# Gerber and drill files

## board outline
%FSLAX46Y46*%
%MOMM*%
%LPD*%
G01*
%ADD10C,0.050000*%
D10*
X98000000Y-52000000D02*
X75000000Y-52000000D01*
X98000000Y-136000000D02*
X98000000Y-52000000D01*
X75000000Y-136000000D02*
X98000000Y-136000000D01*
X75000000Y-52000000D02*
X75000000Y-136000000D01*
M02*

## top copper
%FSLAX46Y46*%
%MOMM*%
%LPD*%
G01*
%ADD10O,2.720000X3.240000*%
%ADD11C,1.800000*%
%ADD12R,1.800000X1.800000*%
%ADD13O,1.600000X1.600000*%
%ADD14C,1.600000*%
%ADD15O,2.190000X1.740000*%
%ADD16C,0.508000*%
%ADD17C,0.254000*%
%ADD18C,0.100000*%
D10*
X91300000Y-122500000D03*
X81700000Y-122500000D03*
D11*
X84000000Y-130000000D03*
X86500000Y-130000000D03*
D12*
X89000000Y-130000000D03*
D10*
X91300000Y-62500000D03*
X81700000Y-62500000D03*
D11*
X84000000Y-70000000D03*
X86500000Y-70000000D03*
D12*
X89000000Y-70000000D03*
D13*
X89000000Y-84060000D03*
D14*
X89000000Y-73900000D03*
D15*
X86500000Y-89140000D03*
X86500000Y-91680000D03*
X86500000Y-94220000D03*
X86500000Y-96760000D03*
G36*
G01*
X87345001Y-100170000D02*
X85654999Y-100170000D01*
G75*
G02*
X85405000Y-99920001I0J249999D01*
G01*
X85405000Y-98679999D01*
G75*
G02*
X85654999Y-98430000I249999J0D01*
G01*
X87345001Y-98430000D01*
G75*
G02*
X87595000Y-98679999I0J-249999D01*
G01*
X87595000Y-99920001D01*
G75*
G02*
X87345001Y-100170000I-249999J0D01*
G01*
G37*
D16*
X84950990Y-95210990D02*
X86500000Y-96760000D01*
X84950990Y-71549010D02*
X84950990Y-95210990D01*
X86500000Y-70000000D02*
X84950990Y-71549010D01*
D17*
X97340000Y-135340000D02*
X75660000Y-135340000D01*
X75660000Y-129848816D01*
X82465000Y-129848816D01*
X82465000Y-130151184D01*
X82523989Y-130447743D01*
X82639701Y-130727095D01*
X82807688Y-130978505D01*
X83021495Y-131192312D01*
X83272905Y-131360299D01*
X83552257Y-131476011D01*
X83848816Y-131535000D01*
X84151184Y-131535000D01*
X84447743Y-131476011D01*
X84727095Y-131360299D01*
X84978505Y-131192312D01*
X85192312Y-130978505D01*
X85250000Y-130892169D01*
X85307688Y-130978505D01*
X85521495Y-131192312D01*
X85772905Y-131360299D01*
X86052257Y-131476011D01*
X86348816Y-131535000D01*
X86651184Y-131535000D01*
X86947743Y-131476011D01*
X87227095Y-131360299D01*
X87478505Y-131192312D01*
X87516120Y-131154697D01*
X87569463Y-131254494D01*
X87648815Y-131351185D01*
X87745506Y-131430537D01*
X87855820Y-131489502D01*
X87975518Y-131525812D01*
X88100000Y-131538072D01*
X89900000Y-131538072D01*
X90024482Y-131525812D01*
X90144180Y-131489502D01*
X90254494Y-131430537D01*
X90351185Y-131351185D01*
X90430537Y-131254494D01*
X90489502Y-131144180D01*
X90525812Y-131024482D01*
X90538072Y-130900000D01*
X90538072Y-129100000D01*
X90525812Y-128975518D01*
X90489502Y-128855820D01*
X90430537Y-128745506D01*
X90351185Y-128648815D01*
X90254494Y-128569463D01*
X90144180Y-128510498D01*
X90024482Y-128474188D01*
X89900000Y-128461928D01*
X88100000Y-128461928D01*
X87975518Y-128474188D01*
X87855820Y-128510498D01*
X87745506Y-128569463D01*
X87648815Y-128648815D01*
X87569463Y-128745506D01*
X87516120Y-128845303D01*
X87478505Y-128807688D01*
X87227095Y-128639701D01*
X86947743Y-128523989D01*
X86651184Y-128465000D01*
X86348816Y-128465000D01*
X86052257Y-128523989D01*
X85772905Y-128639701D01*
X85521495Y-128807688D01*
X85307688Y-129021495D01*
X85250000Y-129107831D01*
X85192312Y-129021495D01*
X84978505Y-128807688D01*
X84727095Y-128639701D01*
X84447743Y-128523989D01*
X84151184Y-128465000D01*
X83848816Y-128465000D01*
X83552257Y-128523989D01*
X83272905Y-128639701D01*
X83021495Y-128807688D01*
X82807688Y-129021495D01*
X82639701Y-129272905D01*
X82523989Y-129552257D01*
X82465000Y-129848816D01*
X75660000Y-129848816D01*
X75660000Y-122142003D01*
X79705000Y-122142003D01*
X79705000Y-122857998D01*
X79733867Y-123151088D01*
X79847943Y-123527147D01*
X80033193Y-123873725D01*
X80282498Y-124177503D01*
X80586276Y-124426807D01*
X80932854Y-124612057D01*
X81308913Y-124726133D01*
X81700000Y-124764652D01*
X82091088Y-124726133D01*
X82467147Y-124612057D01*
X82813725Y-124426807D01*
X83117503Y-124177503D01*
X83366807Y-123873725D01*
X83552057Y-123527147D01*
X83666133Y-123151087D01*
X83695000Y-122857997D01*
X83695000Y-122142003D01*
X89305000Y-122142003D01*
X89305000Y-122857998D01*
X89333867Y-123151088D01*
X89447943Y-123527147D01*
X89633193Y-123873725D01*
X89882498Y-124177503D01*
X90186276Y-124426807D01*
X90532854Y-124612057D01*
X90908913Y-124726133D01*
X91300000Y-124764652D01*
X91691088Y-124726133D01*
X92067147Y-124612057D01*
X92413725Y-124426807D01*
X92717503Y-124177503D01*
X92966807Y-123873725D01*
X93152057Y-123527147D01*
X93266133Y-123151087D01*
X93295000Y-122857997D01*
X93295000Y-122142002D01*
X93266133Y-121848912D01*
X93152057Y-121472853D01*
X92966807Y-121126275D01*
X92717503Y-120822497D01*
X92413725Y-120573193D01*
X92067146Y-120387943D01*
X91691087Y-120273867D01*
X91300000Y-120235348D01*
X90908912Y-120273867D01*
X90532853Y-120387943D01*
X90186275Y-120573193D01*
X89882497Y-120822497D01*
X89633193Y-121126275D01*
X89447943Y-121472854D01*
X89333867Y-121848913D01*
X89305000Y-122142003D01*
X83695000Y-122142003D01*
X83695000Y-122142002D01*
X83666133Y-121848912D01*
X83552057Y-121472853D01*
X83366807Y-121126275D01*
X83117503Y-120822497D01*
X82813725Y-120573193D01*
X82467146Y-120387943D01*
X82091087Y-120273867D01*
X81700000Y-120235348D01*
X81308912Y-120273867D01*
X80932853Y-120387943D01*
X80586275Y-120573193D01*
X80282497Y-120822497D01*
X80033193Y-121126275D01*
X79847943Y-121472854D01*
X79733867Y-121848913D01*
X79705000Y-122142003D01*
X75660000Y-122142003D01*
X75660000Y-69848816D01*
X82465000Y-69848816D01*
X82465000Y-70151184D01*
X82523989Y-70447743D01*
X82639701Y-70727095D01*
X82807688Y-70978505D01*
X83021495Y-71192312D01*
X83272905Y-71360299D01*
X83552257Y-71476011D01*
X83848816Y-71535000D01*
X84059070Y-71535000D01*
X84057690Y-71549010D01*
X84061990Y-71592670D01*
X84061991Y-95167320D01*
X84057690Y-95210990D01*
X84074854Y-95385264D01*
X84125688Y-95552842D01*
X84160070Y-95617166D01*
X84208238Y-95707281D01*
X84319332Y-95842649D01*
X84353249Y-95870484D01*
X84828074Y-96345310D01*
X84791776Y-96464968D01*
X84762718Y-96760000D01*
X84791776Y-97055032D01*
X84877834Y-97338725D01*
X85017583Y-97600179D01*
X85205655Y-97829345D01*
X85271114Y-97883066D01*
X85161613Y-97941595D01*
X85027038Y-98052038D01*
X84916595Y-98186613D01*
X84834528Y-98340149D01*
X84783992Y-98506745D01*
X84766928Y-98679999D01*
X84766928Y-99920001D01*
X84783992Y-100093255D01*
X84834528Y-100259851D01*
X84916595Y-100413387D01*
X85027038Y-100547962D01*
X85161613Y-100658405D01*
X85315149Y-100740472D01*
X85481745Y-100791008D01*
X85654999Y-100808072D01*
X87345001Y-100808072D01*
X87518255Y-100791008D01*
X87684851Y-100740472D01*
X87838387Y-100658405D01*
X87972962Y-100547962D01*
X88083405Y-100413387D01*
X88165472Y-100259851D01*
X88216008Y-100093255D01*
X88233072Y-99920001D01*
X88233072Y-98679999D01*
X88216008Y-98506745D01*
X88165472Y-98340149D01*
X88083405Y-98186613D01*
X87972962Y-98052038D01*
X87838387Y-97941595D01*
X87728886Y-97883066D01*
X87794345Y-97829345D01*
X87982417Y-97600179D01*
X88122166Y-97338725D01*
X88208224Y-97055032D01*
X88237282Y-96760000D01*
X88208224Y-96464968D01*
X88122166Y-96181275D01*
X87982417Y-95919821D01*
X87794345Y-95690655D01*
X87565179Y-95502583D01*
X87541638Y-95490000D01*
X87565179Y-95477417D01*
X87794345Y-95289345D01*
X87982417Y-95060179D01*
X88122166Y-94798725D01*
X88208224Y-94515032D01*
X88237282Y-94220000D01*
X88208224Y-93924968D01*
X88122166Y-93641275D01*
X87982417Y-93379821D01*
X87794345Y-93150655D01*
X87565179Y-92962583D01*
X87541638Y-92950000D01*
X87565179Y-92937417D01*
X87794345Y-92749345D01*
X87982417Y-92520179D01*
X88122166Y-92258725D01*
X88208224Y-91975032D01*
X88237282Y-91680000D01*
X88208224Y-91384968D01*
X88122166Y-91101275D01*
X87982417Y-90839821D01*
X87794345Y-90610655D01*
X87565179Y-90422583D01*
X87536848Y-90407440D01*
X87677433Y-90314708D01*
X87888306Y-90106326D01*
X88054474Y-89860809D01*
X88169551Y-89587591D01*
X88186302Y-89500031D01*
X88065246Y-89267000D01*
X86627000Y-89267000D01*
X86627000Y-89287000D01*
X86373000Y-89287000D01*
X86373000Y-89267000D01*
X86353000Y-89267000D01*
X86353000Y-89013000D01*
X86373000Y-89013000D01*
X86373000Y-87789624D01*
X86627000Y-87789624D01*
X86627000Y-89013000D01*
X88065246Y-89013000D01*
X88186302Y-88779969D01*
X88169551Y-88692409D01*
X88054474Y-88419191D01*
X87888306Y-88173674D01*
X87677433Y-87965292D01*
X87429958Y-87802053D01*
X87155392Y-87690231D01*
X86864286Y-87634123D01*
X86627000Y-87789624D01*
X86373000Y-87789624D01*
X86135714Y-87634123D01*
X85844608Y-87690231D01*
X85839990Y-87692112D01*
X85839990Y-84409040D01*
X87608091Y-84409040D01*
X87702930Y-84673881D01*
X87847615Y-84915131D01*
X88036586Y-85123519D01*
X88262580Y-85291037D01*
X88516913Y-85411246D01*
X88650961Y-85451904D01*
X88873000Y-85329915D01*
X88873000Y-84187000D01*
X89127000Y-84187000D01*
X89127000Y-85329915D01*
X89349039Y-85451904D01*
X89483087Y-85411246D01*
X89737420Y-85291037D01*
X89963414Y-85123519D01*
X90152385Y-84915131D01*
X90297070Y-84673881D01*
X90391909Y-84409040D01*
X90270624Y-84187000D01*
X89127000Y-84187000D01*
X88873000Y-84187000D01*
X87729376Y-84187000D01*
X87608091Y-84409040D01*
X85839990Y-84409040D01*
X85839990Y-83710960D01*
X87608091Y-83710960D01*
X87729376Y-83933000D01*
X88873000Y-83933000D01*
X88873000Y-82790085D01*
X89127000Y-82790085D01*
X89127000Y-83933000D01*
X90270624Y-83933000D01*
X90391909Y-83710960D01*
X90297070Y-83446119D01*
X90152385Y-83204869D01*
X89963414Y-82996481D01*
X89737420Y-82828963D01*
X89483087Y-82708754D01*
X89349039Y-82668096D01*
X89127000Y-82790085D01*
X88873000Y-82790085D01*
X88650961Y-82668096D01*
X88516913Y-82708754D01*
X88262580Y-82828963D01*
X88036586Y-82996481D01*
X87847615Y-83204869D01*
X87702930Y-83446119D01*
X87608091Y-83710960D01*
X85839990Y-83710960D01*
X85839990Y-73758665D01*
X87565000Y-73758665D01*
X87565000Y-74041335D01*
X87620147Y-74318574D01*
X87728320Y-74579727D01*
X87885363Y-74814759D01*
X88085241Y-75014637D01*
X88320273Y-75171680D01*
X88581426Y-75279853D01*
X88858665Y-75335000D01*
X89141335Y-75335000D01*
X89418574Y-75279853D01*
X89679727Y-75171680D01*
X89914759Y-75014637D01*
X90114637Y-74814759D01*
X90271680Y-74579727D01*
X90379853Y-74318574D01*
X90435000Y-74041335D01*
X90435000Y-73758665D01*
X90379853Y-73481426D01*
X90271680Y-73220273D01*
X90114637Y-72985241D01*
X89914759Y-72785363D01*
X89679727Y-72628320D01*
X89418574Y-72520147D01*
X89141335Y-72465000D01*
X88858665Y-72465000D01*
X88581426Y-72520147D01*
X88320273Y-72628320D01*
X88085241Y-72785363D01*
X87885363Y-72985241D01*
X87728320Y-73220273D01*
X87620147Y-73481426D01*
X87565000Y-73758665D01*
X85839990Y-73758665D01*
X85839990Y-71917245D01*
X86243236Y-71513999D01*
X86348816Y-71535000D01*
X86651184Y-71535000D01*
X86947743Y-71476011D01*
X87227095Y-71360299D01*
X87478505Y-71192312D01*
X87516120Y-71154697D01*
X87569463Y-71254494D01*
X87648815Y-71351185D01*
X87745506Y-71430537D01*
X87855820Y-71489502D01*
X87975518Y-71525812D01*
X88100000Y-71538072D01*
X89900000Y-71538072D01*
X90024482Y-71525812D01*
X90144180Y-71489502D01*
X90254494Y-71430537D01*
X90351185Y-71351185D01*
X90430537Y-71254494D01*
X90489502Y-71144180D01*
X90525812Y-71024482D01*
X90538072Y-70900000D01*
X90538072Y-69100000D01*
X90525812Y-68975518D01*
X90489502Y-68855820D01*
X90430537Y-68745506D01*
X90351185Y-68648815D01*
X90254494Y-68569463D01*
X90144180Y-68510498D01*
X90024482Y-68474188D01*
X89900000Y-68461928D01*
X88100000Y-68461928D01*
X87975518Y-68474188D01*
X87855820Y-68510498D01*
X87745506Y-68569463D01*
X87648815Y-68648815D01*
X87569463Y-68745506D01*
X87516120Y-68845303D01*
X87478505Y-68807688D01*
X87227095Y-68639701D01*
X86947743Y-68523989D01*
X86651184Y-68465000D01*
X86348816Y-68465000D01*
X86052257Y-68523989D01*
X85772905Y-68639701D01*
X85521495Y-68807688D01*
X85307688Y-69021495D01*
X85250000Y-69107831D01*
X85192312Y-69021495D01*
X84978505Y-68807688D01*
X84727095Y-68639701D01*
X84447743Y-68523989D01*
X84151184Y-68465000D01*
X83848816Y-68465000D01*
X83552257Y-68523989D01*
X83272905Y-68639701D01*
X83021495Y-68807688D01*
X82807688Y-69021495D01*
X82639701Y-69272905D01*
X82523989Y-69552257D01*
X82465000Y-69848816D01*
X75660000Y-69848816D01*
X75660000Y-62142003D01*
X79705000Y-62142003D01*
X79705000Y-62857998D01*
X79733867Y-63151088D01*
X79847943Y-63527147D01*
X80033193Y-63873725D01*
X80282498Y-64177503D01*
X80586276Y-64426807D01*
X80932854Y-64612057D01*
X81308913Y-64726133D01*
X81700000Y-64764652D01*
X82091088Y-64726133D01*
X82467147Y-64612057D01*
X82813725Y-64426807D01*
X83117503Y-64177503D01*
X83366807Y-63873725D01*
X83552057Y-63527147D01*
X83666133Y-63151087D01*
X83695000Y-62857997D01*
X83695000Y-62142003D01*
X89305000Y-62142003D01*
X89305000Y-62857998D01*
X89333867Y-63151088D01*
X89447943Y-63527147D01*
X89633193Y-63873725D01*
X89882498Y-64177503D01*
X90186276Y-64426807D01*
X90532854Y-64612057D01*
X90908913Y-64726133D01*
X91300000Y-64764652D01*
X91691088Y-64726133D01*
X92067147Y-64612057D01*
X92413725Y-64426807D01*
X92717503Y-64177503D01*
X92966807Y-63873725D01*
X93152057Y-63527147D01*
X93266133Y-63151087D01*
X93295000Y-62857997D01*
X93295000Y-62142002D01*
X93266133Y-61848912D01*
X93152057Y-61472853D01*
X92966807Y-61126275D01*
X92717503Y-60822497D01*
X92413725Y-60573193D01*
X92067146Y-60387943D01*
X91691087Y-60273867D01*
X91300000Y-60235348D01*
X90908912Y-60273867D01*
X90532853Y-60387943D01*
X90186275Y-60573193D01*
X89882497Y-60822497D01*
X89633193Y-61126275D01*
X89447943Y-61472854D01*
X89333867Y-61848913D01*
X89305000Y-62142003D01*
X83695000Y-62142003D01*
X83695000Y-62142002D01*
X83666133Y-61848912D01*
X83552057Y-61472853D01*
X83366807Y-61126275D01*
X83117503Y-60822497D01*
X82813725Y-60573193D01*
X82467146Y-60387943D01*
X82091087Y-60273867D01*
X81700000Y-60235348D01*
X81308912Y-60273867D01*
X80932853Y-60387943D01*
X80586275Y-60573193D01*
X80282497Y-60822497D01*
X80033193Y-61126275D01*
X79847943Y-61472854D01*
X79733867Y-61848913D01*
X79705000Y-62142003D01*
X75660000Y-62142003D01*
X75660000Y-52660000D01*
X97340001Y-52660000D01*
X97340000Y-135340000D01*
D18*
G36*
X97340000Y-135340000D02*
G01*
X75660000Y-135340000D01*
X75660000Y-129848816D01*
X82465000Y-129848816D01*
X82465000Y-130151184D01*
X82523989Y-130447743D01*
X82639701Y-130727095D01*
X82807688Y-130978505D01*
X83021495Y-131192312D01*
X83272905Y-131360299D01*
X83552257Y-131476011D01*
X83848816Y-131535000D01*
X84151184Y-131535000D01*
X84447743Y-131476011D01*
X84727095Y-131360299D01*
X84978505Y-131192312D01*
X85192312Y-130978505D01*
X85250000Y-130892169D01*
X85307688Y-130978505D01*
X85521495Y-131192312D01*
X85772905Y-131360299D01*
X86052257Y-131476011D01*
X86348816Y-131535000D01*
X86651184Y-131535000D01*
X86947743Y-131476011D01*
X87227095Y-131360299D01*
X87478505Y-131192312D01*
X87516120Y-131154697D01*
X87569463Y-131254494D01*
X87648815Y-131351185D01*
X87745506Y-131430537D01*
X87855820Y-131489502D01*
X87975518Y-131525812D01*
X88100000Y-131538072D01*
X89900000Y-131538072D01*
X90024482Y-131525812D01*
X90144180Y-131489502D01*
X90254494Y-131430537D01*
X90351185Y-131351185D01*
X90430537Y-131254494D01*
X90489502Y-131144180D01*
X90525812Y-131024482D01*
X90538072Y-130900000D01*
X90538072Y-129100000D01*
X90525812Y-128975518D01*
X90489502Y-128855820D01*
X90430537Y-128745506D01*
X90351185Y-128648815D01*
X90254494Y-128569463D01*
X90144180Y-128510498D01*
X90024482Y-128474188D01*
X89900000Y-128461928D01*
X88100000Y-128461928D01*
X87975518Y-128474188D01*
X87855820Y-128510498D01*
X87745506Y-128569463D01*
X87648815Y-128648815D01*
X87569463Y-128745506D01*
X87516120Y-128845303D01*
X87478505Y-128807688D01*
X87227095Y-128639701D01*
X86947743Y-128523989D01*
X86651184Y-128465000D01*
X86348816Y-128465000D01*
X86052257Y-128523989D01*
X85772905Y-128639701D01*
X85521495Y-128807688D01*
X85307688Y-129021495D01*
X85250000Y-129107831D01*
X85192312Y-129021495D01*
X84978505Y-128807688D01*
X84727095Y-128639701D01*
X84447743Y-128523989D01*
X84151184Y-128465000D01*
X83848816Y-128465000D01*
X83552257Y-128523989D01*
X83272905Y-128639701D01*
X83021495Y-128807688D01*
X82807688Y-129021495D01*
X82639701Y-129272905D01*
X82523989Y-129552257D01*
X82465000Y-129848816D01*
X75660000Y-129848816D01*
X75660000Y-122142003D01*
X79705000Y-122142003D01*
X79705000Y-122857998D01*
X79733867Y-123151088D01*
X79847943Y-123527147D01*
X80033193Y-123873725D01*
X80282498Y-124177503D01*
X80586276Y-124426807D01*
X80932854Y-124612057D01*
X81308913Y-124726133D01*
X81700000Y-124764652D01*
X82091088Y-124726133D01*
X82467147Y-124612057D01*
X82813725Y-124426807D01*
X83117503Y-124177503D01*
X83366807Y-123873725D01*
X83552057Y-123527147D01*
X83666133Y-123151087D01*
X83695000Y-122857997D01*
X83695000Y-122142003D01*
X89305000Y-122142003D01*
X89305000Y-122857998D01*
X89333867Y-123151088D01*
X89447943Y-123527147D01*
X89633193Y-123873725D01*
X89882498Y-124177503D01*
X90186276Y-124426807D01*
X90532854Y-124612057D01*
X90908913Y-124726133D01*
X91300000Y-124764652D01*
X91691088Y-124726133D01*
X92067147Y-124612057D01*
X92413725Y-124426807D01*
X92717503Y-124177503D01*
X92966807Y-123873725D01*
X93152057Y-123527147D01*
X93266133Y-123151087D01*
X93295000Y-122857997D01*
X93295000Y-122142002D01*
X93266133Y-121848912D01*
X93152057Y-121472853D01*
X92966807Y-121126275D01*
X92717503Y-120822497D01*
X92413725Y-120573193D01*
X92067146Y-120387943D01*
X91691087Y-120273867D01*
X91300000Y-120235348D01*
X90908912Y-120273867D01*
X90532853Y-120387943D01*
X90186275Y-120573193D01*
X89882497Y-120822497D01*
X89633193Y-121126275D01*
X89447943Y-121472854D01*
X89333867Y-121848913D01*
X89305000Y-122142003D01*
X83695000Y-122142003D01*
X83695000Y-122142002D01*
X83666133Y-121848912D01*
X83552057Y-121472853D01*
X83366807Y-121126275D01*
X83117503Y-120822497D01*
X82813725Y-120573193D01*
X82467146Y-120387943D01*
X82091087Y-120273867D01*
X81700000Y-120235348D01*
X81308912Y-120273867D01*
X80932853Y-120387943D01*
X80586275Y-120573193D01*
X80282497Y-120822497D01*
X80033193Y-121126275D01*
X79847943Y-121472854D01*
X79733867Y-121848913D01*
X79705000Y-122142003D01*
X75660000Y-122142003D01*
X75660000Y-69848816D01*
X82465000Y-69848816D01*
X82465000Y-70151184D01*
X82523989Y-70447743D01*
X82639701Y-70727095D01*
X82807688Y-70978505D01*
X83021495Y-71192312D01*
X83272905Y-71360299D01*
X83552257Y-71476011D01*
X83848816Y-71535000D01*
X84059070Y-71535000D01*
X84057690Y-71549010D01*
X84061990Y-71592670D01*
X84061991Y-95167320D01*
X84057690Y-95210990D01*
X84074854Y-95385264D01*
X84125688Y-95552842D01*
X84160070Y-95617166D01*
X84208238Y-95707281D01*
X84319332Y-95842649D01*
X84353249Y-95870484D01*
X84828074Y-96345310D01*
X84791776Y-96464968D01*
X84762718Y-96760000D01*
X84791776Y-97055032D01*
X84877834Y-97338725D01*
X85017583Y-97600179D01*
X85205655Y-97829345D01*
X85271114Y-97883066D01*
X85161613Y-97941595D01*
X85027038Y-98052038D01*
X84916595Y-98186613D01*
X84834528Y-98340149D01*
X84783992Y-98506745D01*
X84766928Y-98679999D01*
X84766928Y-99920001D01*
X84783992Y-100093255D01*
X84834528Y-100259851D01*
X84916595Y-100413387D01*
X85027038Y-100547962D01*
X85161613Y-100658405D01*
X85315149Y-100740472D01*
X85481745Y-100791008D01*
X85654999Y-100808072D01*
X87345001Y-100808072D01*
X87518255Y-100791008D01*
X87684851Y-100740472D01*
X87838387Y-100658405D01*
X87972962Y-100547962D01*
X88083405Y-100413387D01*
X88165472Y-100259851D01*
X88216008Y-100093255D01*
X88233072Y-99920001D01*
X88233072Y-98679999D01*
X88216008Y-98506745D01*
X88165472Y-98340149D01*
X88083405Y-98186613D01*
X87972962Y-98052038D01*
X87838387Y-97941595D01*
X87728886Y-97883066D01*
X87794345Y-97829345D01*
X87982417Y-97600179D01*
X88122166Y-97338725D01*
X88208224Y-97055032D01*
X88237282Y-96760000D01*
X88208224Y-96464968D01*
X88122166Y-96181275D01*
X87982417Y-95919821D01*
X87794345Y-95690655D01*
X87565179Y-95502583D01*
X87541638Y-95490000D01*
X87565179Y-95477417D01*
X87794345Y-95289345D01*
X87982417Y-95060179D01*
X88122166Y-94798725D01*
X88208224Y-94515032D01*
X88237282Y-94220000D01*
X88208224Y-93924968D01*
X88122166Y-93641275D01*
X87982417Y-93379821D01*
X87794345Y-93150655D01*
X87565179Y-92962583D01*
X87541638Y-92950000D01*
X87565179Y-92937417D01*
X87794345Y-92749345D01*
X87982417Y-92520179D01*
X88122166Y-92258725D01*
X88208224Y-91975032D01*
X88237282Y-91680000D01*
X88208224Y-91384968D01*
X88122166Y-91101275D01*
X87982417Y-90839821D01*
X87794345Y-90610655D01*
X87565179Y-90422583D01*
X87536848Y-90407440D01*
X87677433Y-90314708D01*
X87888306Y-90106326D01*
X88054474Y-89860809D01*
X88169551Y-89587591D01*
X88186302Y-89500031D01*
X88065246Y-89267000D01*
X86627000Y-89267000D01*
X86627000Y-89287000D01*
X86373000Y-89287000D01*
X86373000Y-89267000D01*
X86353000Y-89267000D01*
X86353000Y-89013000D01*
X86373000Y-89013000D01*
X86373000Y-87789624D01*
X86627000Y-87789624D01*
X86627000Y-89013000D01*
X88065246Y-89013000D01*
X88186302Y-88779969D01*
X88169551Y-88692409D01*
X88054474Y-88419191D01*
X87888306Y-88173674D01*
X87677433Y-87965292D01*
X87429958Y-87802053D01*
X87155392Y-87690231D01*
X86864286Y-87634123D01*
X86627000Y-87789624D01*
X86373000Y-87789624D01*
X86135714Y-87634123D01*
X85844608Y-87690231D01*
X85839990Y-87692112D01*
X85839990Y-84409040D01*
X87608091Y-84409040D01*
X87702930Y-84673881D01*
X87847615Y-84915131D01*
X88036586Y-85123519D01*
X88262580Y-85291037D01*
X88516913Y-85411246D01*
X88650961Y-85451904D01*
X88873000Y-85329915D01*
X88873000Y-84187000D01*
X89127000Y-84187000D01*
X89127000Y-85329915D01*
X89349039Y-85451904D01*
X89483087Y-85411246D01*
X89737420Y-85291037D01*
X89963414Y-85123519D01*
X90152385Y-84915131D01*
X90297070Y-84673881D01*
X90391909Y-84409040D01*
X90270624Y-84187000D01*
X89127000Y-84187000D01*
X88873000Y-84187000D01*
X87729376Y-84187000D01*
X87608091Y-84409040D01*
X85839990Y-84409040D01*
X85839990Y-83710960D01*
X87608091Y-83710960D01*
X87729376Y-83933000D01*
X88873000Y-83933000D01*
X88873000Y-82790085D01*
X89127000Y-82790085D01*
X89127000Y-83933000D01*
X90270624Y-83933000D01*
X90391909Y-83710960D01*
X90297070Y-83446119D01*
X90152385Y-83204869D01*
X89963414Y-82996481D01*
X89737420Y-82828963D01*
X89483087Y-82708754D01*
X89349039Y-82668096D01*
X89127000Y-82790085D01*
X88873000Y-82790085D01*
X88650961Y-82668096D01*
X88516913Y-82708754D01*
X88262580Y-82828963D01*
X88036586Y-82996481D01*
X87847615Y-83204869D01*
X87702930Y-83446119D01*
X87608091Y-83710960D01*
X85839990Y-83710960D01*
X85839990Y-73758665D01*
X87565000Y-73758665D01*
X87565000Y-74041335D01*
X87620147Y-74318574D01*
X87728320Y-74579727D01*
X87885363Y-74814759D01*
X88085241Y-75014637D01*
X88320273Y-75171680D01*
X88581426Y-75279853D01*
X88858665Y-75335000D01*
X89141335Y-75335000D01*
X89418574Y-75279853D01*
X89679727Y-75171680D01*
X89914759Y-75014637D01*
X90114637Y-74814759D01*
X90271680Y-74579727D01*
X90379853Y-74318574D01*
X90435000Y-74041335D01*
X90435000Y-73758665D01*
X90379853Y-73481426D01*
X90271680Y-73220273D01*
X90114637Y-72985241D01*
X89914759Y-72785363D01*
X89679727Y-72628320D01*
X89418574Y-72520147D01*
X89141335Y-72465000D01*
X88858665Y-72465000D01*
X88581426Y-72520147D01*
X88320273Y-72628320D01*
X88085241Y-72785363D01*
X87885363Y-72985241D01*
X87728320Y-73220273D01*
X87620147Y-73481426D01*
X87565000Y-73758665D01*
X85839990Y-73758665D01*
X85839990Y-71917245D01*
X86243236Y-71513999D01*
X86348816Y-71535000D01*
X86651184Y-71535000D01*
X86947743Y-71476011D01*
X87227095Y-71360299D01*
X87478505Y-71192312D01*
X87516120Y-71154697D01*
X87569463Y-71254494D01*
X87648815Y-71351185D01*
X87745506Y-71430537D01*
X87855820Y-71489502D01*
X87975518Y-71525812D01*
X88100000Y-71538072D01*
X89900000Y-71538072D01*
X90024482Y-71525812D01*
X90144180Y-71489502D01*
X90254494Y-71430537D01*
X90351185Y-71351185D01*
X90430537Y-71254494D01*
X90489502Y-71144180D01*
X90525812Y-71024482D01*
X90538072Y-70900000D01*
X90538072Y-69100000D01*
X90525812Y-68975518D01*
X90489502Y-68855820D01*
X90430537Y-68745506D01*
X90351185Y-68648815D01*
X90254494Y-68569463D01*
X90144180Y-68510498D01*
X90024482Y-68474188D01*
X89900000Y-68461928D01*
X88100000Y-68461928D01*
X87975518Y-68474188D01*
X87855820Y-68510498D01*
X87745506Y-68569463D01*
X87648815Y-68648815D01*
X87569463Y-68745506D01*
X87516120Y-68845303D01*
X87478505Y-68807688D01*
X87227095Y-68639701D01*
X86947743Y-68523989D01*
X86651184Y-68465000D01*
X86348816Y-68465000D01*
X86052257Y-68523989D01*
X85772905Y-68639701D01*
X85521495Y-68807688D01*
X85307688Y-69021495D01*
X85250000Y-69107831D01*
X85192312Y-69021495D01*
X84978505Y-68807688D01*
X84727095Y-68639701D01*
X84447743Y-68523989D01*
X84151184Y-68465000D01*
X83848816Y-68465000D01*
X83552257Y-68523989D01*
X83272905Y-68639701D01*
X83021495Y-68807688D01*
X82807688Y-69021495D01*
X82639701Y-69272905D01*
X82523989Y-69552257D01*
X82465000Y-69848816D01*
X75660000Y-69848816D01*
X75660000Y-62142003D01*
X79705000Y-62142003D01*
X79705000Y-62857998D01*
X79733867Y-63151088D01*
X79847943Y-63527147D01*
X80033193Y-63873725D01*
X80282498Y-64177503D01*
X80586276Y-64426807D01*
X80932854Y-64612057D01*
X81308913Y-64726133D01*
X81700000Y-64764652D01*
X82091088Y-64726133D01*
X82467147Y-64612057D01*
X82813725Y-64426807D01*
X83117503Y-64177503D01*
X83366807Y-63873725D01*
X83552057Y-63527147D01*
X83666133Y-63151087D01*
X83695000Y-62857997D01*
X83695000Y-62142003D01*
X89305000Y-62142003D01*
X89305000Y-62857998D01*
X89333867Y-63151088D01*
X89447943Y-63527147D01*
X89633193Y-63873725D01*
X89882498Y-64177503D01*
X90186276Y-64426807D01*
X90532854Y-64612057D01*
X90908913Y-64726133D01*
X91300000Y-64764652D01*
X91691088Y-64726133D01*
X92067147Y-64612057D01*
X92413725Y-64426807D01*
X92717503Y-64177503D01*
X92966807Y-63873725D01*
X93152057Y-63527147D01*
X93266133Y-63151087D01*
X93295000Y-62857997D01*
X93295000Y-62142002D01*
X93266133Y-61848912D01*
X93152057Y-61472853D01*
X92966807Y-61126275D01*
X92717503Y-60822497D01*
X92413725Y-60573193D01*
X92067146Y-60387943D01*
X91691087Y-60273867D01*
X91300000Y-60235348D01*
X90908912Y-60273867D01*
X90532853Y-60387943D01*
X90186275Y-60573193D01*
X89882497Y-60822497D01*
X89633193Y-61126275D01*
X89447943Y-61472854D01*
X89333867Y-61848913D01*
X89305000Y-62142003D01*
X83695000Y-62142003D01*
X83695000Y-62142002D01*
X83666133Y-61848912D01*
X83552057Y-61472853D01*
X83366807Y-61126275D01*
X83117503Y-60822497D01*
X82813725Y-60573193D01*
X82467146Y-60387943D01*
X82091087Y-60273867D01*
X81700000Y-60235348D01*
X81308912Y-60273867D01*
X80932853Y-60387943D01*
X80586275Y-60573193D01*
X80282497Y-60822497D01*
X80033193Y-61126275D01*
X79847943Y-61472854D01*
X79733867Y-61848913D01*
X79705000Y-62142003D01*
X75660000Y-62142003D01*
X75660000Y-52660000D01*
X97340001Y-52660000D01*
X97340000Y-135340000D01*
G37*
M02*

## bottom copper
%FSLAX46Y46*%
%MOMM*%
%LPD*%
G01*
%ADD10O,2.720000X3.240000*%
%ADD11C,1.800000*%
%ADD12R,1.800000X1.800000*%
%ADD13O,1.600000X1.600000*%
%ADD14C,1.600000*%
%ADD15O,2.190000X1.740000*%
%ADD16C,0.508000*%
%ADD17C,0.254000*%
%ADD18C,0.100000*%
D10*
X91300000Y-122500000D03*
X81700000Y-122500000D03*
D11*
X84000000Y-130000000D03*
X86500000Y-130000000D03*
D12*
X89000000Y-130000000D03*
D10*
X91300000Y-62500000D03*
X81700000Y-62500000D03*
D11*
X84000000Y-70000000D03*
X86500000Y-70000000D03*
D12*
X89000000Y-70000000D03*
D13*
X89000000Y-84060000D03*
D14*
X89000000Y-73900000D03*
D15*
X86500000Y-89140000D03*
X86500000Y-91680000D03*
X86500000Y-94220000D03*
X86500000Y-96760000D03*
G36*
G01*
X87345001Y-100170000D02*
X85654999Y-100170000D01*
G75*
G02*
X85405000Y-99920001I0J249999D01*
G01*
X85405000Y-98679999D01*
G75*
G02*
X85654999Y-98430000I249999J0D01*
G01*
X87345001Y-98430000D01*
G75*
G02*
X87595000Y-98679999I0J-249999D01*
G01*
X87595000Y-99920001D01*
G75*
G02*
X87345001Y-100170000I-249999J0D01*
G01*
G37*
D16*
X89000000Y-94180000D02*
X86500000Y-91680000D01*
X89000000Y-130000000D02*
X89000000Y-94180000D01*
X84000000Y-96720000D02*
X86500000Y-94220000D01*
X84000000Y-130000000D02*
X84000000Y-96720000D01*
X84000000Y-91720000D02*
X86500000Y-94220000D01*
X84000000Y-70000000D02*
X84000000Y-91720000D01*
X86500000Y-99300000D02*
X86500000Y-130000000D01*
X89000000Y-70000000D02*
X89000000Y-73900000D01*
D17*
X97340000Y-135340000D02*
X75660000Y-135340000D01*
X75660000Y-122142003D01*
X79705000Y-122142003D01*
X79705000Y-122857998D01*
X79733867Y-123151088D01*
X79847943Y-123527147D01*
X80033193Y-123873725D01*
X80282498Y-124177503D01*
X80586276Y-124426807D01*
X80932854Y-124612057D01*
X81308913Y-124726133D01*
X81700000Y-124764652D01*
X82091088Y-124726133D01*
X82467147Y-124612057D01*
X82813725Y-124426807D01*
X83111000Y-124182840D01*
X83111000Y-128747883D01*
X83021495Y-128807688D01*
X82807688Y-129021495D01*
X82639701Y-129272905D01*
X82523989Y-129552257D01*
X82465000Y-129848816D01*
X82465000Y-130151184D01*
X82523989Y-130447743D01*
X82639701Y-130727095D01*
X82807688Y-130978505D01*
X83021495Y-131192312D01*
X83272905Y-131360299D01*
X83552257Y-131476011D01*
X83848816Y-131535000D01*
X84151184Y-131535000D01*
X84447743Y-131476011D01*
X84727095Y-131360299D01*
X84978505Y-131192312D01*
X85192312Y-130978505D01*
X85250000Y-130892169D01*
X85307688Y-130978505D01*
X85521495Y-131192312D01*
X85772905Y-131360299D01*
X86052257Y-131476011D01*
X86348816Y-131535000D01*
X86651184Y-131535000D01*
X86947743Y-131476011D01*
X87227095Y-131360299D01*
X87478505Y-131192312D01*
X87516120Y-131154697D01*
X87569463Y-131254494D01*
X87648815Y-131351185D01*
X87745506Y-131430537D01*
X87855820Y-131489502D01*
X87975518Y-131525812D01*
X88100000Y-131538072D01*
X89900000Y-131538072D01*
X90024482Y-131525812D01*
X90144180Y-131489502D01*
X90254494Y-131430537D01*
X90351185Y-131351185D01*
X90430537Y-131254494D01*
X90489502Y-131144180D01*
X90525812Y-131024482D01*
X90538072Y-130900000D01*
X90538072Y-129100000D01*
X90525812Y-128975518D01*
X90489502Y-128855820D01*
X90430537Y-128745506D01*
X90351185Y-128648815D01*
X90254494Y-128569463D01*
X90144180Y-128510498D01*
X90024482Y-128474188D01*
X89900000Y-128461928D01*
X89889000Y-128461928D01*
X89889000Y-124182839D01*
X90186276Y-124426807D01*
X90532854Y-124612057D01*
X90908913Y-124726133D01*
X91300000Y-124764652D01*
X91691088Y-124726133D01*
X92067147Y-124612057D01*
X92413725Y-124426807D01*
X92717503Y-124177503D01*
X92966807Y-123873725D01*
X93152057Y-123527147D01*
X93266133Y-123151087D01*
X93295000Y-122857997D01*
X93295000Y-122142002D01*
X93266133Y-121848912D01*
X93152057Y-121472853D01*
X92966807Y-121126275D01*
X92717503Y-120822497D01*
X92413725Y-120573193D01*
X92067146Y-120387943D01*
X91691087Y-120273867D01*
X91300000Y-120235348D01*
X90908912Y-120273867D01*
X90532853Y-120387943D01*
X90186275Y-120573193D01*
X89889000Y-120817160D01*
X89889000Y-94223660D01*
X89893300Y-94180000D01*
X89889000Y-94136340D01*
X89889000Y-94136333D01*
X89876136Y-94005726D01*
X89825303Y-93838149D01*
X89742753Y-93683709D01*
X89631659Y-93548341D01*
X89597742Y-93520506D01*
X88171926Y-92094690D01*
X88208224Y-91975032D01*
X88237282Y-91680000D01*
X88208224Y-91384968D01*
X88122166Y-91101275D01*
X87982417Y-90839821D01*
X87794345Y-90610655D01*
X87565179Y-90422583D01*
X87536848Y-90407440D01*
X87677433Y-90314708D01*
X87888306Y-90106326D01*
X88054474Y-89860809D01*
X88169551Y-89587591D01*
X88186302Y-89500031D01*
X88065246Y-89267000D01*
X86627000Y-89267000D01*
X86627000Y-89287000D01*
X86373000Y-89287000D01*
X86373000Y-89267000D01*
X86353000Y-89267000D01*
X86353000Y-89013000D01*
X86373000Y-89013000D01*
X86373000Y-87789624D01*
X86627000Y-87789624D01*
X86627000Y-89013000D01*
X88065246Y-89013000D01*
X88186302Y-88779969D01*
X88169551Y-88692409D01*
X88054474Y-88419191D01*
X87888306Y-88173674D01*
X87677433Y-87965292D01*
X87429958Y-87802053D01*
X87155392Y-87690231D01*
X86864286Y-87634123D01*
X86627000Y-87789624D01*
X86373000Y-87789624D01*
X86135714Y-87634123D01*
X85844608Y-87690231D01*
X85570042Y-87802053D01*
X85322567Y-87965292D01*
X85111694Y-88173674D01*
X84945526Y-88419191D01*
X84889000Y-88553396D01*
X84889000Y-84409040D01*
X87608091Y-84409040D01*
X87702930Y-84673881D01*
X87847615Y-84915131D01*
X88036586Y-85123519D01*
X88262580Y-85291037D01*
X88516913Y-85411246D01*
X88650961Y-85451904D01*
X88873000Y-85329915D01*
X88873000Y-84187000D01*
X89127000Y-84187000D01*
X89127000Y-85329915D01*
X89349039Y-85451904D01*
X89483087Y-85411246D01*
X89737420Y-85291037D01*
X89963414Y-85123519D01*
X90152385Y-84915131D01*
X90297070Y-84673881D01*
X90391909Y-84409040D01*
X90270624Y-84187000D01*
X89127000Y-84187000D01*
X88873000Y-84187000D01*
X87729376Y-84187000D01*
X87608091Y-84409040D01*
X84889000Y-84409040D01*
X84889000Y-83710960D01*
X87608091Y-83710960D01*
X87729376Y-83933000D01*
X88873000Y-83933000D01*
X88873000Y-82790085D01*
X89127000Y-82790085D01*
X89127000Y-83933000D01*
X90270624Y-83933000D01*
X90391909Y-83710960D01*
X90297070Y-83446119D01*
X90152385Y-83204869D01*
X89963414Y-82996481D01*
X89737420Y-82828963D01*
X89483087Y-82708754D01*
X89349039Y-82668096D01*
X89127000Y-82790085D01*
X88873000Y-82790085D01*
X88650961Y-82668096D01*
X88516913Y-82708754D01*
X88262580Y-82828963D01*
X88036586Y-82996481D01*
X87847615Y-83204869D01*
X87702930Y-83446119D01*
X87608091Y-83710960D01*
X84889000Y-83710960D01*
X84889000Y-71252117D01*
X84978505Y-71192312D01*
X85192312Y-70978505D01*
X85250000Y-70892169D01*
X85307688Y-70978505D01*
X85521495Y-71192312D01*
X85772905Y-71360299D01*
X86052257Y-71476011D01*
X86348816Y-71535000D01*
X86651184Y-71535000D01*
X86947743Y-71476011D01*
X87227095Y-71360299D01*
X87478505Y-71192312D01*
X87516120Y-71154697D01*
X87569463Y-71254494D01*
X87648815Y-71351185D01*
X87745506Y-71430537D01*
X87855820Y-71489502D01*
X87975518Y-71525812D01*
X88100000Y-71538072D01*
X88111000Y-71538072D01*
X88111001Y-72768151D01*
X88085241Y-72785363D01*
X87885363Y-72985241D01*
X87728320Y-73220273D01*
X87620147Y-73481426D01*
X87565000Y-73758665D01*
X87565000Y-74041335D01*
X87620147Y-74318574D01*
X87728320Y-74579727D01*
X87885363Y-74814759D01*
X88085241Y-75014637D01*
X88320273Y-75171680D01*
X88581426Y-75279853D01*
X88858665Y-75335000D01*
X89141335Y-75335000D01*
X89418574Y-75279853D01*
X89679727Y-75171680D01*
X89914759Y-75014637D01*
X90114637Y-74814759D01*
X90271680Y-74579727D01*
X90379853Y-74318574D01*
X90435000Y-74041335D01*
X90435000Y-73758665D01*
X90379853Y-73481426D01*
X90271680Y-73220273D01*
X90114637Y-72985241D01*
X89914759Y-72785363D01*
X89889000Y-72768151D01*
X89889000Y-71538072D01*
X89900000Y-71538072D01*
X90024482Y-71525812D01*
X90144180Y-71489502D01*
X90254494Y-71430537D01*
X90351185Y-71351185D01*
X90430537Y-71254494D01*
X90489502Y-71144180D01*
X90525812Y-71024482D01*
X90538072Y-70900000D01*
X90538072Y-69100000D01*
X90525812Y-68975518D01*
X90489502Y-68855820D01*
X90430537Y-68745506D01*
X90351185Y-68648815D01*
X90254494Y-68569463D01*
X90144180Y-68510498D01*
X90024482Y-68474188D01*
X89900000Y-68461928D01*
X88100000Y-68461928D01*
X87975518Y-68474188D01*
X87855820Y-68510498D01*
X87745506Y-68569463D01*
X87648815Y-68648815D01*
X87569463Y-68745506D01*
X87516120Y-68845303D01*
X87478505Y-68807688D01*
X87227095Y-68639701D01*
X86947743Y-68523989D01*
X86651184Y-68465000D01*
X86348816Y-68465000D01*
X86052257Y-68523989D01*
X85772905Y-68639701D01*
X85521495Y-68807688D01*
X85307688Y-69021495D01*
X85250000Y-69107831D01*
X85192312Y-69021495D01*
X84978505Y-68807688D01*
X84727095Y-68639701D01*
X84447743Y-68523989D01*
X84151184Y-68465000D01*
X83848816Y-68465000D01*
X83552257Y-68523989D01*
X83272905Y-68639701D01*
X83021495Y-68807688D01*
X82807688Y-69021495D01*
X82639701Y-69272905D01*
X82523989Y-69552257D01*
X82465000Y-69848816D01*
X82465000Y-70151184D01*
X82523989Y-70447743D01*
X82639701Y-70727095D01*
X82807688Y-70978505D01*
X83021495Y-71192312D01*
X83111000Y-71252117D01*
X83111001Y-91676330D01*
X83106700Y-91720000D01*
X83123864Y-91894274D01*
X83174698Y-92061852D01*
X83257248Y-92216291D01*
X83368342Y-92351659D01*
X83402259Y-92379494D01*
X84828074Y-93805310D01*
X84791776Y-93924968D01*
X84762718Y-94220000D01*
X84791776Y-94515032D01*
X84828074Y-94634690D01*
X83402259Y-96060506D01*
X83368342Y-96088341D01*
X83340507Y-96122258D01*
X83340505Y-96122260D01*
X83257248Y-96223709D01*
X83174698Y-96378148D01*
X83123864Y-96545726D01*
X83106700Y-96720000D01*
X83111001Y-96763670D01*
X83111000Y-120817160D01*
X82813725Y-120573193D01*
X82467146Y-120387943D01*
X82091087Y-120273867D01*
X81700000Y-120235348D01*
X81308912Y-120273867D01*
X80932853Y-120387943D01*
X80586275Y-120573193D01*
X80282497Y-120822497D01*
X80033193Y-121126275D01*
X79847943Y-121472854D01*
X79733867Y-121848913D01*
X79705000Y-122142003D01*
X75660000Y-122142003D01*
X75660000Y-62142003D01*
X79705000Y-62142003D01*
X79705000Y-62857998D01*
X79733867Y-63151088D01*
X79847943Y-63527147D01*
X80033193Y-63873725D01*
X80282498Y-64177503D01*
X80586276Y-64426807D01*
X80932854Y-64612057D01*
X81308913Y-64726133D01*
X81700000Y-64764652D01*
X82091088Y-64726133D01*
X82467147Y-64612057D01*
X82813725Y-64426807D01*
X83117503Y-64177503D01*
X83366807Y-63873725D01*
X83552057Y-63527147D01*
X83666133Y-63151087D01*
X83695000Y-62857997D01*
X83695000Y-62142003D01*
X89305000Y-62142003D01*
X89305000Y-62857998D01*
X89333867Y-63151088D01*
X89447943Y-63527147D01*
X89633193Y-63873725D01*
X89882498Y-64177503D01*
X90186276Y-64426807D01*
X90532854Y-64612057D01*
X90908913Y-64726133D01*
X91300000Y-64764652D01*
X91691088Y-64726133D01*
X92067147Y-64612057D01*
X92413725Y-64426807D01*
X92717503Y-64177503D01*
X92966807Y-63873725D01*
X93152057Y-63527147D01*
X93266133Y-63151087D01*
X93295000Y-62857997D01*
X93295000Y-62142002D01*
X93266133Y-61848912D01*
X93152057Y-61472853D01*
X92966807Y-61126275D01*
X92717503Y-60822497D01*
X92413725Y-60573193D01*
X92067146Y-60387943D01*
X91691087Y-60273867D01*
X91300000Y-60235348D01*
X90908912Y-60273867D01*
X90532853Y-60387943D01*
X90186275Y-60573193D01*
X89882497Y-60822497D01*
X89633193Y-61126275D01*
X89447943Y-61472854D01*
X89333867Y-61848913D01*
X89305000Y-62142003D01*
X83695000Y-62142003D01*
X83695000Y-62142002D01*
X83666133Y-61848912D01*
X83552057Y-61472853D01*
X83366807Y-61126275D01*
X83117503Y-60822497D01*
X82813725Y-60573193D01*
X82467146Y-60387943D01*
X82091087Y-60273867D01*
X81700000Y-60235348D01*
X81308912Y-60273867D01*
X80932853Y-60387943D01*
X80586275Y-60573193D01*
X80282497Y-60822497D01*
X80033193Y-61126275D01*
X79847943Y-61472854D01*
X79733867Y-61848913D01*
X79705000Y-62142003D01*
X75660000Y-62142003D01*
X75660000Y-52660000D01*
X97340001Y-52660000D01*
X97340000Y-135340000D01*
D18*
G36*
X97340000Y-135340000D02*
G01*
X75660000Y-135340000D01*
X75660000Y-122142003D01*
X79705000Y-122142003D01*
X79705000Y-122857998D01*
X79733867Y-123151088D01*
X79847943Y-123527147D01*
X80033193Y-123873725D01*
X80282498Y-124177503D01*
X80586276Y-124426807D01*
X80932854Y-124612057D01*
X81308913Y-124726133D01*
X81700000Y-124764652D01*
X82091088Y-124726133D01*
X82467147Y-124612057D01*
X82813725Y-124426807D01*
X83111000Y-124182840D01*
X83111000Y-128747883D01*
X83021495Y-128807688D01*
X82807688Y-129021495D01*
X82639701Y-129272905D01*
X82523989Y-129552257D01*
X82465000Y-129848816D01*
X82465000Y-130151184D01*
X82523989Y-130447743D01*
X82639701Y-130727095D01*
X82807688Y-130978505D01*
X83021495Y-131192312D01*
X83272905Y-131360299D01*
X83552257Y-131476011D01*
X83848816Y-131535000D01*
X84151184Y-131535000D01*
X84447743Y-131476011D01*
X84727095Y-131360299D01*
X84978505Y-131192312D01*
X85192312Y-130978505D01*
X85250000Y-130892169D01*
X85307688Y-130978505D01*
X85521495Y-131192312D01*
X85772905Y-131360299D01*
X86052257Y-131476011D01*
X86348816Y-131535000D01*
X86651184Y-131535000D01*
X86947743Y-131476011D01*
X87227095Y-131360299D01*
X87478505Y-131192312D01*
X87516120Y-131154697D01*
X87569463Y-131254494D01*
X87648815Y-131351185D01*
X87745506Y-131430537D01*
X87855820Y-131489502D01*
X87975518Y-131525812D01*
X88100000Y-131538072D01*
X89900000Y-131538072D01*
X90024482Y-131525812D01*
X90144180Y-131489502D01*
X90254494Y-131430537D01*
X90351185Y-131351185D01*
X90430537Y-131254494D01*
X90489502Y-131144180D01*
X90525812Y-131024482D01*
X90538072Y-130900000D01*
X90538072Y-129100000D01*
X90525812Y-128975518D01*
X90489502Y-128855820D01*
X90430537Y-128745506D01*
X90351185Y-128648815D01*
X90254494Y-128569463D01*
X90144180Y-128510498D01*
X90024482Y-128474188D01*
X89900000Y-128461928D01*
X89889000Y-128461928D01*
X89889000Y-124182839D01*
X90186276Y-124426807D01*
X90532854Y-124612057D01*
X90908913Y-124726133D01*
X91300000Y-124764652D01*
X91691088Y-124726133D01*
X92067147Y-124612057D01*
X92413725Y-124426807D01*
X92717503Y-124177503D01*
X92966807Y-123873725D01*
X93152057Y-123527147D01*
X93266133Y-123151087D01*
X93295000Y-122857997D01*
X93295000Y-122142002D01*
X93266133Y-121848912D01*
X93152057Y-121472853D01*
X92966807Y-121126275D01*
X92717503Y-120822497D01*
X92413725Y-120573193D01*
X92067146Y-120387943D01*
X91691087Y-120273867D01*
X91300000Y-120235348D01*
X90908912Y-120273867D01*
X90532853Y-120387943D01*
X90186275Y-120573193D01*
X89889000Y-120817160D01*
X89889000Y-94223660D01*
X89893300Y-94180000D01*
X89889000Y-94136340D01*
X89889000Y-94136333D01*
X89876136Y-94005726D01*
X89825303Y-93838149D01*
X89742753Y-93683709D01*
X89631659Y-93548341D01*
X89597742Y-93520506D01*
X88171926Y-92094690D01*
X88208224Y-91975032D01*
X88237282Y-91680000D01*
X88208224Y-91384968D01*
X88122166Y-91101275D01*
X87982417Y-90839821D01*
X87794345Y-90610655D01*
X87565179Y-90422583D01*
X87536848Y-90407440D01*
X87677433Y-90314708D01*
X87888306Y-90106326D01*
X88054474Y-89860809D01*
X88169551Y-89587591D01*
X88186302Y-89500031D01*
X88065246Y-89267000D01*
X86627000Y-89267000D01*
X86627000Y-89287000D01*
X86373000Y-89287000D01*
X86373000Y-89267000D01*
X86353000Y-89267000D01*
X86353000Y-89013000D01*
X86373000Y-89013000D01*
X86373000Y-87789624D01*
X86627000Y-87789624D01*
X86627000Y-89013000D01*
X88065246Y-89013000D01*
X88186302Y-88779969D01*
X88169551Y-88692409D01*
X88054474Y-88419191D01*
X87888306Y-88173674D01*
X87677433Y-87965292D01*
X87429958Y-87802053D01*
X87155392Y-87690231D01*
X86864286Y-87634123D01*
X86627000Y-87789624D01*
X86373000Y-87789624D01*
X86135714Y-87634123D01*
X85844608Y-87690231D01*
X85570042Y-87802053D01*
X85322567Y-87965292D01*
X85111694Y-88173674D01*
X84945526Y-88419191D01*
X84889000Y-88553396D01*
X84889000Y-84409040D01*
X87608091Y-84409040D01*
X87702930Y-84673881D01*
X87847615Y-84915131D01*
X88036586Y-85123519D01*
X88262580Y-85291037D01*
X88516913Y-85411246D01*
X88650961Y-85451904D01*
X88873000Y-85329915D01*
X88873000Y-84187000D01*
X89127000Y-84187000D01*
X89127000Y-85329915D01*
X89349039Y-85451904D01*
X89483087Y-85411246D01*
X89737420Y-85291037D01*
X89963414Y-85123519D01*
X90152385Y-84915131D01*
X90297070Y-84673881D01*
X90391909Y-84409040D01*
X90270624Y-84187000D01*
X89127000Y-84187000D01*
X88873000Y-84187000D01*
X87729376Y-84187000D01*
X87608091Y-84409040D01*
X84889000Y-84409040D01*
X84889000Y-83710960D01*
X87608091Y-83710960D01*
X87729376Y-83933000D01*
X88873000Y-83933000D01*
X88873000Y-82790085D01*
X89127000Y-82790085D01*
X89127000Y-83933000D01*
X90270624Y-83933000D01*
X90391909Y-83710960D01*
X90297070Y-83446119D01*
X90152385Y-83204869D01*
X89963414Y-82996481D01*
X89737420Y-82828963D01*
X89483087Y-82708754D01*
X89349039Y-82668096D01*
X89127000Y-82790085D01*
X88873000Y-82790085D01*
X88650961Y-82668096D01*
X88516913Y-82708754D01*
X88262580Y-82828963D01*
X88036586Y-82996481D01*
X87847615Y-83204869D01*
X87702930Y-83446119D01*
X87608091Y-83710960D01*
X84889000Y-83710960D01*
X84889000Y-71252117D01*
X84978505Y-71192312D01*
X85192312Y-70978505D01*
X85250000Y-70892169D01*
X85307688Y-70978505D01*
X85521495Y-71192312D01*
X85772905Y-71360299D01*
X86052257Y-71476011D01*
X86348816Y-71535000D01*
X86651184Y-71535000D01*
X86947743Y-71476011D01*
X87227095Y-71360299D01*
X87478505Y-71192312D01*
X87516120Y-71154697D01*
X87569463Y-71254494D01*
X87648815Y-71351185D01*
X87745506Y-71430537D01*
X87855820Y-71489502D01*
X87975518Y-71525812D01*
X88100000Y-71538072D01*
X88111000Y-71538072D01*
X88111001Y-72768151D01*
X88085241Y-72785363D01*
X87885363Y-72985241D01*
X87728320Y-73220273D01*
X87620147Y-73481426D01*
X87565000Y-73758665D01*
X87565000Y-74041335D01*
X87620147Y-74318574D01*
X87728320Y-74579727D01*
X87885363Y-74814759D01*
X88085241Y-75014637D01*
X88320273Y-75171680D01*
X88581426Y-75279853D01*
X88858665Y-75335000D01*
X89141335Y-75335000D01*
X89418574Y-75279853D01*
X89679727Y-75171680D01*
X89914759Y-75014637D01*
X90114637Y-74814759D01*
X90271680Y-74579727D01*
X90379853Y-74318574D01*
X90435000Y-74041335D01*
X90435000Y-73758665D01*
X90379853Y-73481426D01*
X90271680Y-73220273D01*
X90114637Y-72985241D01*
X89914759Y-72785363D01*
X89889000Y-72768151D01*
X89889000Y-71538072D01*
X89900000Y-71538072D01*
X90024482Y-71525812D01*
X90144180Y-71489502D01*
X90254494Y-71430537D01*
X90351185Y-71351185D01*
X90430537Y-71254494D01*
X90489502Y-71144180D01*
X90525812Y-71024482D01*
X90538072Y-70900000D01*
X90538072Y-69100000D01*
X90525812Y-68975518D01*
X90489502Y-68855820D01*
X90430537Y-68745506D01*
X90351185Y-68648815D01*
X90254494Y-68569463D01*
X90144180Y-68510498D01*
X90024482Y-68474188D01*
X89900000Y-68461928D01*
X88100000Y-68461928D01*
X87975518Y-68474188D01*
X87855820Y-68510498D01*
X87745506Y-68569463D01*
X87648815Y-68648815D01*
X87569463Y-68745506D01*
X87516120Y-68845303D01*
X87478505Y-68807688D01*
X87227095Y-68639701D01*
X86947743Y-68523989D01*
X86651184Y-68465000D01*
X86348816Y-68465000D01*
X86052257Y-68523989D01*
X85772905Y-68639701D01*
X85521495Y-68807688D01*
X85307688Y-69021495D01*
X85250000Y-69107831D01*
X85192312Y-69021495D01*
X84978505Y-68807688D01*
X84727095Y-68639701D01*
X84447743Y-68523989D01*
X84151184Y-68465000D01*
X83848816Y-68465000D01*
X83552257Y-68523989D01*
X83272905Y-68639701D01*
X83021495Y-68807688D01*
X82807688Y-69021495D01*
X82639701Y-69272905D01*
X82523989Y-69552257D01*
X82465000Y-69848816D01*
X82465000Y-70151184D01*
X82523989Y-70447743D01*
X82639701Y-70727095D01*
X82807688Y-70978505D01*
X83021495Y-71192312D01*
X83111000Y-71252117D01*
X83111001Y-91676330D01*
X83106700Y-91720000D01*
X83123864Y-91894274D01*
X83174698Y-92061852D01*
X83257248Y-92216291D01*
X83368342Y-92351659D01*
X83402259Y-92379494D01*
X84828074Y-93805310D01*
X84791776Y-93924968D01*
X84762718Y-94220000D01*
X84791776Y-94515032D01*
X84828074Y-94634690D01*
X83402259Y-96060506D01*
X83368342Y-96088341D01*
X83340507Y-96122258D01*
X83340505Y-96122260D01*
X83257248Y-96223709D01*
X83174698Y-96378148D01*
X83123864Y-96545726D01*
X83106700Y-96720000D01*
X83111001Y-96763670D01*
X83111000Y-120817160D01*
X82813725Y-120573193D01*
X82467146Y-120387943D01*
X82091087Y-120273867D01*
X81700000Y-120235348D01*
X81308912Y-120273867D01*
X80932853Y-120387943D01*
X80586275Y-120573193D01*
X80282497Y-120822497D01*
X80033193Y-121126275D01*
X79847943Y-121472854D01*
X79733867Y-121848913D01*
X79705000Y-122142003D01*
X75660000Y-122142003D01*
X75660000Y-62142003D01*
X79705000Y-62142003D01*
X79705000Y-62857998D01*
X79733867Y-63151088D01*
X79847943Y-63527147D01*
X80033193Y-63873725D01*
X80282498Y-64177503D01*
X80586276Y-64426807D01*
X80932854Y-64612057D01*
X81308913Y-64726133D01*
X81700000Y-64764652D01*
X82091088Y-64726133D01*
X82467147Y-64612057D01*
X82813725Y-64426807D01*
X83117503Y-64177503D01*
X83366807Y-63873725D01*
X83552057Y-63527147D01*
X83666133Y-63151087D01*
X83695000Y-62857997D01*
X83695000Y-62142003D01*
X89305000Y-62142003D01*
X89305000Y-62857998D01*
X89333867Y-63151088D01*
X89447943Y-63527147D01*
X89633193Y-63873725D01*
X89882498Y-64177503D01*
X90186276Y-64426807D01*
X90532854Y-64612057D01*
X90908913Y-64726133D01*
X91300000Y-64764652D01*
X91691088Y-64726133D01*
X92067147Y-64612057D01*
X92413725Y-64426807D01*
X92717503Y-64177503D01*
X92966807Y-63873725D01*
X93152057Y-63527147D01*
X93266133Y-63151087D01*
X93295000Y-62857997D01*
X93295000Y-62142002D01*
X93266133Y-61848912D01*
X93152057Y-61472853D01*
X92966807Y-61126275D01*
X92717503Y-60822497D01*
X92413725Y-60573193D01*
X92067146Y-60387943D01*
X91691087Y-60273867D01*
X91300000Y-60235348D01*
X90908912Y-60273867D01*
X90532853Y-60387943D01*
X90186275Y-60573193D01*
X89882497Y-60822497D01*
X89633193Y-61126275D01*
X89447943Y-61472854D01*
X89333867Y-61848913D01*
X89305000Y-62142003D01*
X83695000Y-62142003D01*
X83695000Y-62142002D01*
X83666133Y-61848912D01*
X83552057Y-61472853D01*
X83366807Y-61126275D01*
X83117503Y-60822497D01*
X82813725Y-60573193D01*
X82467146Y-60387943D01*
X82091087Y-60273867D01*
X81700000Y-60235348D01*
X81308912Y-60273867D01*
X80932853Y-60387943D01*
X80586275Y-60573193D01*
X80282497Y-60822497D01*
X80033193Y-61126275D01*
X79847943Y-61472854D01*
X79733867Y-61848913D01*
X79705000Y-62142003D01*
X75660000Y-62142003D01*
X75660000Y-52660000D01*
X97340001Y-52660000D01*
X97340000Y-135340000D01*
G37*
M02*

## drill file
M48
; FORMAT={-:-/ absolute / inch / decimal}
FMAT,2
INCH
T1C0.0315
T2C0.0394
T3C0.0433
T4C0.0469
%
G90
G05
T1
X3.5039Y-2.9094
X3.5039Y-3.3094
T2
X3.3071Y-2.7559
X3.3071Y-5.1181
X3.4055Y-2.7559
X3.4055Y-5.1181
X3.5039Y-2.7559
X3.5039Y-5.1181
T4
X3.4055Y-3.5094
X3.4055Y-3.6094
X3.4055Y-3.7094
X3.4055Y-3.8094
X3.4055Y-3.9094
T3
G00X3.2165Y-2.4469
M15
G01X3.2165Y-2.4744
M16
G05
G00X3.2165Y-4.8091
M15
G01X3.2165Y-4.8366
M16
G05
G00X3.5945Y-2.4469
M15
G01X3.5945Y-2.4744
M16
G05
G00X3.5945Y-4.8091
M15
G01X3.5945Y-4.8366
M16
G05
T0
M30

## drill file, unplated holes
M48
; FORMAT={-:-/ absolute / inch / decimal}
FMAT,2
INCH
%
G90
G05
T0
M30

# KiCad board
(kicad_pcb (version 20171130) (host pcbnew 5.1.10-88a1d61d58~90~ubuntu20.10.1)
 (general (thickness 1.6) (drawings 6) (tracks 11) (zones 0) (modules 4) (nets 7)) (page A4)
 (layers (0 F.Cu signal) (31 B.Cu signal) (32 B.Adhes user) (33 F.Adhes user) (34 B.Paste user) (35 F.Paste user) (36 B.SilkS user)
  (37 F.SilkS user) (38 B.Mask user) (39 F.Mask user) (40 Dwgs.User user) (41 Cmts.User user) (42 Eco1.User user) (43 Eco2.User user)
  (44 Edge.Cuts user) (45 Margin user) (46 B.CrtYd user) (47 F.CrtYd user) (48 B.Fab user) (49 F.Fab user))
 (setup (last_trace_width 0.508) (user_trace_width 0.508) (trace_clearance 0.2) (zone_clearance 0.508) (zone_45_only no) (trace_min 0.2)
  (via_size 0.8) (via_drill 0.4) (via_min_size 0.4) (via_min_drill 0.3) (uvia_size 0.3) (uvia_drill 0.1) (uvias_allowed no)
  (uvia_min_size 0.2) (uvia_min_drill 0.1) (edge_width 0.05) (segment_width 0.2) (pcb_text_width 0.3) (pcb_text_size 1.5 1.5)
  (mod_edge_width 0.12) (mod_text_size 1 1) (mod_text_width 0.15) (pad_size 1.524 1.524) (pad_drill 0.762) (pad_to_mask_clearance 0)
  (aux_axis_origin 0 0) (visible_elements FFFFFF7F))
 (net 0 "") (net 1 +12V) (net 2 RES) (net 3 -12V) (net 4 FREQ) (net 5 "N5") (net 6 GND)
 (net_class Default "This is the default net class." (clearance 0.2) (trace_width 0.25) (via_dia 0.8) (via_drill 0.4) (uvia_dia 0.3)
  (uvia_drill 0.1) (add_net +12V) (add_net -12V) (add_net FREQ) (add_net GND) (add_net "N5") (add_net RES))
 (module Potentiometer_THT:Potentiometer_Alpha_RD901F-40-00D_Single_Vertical (layer B.Cu) (at 89 130 90)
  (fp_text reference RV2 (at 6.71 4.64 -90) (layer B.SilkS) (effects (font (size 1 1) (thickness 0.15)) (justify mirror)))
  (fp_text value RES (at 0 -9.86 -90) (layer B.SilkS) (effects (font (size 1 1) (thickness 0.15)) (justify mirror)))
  (pad "" thru_hole oval (at 7.5 2.3) (size 2.72 3.24) (drill oval 1.1 1.8) (layers *.Cu *.Mask))
  (pad "" thru_hole oval (at 7.5 -7.3) (size 2.72 3.24) (drill oval 1.1 1.8) (layers *.Cu *.Mask))
  (pad 3 thru_hole circle (at 0 -5) (size 1.8 1.8) (drill 1) (layers *.Cu *.Mask) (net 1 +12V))
  (pad 2 thru_hole circle (at 0 -2.5) (size 1.8 1.8) (drill 1) (layers *.Cu *.Mask) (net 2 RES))
  (pad 1 thru_hole rect (at 0 0) (size 1.8 1.8) (drill 1) (layers *.Cu *.Mask) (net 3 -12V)))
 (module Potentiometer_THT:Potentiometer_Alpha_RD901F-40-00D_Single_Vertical (layer B.Cu) (at 89 70 90)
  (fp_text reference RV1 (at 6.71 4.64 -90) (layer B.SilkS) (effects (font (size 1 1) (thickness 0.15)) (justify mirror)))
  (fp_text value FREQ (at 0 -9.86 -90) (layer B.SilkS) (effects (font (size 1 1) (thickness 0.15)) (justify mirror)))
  (pad "" thru_hole oval (at 7.5 2.3) (size 2.72 3.24) (drill oval 1.1 1.8) (layers *.Cu *.Mask))
  (pad "" thru_hole oval (at 7.5 -7.3) (size 2.72 3.24) (drill oval 1.1 1.8) (layers *.Cu *.Mask))
  (pad 3 thru_hole circle (at 0 -5) (size 1.8 1.8) (drill 1) (layers *.Cu *.Mask) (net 1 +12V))
  (pad 2 thru_hole circle (at 0 -2.5) (size 1.8 1.8) (drill 1) (layers *.Cu *.Mask) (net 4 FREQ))
  (pad 1 thru_hole rect (at 0 0) (size 1.8 1.8) (drill 1) (layers *.Cu *.Mask) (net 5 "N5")))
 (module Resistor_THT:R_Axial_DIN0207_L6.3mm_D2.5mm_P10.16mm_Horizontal (layer F.Cu) (at 89 73.9 270)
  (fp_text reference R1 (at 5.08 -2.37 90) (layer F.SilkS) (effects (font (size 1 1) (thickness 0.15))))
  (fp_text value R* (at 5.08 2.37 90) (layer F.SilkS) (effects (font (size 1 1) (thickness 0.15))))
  (pad 2 thru_hole oval (at 10.16 0 270) (size 1.6 1.6) (drill 0.8) (layers *.Cu *.Mask) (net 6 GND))
  (pad 1 thru_hole circle (at 0 0 270) (size 1.6 1.6) (drill 0.8) (layers *.Cu *.Mask) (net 5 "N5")))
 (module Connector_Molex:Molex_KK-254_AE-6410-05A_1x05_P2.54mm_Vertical (layer F.Cu) (at 86.5 99.3 90)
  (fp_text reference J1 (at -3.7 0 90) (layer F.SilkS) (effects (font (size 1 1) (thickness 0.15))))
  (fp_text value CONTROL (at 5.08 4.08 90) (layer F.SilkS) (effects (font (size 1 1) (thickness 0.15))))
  (pad 5 thru_hole oval (at 10.16 0 90) (size 1.74 2.19) (drill 1.19) (layers *.Cu *.Mask) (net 6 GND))
  (pad 4 thru_hole oval (at 7.62 0 90) (size 1.74 2.19) (drill 1.19) (layers *.Cu *.Mask) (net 3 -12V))
  (pad 3 thru_hole oval (at 5.08 0 90) (size 1.74 2.19) (drill 1.19) (layers *.Cu *.Mask) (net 1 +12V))
  (pad 2 thru_hole oval (at 2.54 0 90) (size 1.74 2.19) (drill 1.19) (layers *.Cu *.Mask) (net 4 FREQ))
  (pad 1 thru_hole roundrect (at 0 0 90) (size 1.74 2.19) (drill 1.19) (layers *.Cu *.Mask) (roundrect_rratio 0.1436775862068966)
   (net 2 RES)))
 (gr_line (start 98 52) (end 75 52) (layer Edge.Cuts) (width 0.05))
 (gr_line (start 98 136) (end 98 52) (layer Edge.Cuts) (width 0.05))
 (gr_line (start 75 136) (end 98 136) (layer Edge.Cuts) (width 0.05))
 (gr_line (start 75 52) (end 75 136) (layer Edge.Cuts) (width 0.05))
 (segment (start 89 94.18) (end 86.5 91.68) (width 0.508) (layer B.Cu) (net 3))
 (segment (start 89 130) (end 89 94.18) (width 0.508) (layer B.Cu) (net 3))
 (segment (start 84 96.72) (end 86.5 94.22) (width 0.508) (layer B.Cu) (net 1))
 (segment (start 84 130) (end 84 96.72) (width 0.508) (layer B.Cu) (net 1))
 (segment (start 84 91.72) (end 86.5 94.22) (width 0.508) (layer B.Cu) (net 1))
 (segment (start 84 70) (end 84 91.72) (width 0.508) (layer B.Cu) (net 1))
 (segment (start 84.95099 95.21099) (end 86.5 96.76) (width 0.508) (layer F.Cu) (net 4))
 (segment (start 84.95099 71.54901) (end 84.95099 95.21099) (width 0.508) (layer F.Cu) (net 4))
 (segment (start 86.5 70) (end 84.95099 71.54901) (width 0.508) (layer F.Cu) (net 4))
 (segment (start 86.5 99.3) (end 86.5 130) (width 0.508) (layer B.Cu) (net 2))
 (segment (start 89 70) (end 89 73.9) (width 0.508) (layer B.Cu) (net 5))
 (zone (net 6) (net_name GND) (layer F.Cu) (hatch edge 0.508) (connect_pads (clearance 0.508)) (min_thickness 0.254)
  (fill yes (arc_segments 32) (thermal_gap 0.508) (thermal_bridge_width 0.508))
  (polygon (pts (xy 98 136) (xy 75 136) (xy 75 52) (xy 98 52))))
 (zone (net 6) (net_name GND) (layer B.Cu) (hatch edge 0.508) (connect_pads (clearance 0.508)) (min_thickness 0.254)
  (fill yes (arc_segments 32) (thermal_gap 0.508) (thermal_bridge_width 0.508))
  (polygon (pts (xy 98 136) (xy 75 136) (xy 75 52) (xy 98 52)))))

